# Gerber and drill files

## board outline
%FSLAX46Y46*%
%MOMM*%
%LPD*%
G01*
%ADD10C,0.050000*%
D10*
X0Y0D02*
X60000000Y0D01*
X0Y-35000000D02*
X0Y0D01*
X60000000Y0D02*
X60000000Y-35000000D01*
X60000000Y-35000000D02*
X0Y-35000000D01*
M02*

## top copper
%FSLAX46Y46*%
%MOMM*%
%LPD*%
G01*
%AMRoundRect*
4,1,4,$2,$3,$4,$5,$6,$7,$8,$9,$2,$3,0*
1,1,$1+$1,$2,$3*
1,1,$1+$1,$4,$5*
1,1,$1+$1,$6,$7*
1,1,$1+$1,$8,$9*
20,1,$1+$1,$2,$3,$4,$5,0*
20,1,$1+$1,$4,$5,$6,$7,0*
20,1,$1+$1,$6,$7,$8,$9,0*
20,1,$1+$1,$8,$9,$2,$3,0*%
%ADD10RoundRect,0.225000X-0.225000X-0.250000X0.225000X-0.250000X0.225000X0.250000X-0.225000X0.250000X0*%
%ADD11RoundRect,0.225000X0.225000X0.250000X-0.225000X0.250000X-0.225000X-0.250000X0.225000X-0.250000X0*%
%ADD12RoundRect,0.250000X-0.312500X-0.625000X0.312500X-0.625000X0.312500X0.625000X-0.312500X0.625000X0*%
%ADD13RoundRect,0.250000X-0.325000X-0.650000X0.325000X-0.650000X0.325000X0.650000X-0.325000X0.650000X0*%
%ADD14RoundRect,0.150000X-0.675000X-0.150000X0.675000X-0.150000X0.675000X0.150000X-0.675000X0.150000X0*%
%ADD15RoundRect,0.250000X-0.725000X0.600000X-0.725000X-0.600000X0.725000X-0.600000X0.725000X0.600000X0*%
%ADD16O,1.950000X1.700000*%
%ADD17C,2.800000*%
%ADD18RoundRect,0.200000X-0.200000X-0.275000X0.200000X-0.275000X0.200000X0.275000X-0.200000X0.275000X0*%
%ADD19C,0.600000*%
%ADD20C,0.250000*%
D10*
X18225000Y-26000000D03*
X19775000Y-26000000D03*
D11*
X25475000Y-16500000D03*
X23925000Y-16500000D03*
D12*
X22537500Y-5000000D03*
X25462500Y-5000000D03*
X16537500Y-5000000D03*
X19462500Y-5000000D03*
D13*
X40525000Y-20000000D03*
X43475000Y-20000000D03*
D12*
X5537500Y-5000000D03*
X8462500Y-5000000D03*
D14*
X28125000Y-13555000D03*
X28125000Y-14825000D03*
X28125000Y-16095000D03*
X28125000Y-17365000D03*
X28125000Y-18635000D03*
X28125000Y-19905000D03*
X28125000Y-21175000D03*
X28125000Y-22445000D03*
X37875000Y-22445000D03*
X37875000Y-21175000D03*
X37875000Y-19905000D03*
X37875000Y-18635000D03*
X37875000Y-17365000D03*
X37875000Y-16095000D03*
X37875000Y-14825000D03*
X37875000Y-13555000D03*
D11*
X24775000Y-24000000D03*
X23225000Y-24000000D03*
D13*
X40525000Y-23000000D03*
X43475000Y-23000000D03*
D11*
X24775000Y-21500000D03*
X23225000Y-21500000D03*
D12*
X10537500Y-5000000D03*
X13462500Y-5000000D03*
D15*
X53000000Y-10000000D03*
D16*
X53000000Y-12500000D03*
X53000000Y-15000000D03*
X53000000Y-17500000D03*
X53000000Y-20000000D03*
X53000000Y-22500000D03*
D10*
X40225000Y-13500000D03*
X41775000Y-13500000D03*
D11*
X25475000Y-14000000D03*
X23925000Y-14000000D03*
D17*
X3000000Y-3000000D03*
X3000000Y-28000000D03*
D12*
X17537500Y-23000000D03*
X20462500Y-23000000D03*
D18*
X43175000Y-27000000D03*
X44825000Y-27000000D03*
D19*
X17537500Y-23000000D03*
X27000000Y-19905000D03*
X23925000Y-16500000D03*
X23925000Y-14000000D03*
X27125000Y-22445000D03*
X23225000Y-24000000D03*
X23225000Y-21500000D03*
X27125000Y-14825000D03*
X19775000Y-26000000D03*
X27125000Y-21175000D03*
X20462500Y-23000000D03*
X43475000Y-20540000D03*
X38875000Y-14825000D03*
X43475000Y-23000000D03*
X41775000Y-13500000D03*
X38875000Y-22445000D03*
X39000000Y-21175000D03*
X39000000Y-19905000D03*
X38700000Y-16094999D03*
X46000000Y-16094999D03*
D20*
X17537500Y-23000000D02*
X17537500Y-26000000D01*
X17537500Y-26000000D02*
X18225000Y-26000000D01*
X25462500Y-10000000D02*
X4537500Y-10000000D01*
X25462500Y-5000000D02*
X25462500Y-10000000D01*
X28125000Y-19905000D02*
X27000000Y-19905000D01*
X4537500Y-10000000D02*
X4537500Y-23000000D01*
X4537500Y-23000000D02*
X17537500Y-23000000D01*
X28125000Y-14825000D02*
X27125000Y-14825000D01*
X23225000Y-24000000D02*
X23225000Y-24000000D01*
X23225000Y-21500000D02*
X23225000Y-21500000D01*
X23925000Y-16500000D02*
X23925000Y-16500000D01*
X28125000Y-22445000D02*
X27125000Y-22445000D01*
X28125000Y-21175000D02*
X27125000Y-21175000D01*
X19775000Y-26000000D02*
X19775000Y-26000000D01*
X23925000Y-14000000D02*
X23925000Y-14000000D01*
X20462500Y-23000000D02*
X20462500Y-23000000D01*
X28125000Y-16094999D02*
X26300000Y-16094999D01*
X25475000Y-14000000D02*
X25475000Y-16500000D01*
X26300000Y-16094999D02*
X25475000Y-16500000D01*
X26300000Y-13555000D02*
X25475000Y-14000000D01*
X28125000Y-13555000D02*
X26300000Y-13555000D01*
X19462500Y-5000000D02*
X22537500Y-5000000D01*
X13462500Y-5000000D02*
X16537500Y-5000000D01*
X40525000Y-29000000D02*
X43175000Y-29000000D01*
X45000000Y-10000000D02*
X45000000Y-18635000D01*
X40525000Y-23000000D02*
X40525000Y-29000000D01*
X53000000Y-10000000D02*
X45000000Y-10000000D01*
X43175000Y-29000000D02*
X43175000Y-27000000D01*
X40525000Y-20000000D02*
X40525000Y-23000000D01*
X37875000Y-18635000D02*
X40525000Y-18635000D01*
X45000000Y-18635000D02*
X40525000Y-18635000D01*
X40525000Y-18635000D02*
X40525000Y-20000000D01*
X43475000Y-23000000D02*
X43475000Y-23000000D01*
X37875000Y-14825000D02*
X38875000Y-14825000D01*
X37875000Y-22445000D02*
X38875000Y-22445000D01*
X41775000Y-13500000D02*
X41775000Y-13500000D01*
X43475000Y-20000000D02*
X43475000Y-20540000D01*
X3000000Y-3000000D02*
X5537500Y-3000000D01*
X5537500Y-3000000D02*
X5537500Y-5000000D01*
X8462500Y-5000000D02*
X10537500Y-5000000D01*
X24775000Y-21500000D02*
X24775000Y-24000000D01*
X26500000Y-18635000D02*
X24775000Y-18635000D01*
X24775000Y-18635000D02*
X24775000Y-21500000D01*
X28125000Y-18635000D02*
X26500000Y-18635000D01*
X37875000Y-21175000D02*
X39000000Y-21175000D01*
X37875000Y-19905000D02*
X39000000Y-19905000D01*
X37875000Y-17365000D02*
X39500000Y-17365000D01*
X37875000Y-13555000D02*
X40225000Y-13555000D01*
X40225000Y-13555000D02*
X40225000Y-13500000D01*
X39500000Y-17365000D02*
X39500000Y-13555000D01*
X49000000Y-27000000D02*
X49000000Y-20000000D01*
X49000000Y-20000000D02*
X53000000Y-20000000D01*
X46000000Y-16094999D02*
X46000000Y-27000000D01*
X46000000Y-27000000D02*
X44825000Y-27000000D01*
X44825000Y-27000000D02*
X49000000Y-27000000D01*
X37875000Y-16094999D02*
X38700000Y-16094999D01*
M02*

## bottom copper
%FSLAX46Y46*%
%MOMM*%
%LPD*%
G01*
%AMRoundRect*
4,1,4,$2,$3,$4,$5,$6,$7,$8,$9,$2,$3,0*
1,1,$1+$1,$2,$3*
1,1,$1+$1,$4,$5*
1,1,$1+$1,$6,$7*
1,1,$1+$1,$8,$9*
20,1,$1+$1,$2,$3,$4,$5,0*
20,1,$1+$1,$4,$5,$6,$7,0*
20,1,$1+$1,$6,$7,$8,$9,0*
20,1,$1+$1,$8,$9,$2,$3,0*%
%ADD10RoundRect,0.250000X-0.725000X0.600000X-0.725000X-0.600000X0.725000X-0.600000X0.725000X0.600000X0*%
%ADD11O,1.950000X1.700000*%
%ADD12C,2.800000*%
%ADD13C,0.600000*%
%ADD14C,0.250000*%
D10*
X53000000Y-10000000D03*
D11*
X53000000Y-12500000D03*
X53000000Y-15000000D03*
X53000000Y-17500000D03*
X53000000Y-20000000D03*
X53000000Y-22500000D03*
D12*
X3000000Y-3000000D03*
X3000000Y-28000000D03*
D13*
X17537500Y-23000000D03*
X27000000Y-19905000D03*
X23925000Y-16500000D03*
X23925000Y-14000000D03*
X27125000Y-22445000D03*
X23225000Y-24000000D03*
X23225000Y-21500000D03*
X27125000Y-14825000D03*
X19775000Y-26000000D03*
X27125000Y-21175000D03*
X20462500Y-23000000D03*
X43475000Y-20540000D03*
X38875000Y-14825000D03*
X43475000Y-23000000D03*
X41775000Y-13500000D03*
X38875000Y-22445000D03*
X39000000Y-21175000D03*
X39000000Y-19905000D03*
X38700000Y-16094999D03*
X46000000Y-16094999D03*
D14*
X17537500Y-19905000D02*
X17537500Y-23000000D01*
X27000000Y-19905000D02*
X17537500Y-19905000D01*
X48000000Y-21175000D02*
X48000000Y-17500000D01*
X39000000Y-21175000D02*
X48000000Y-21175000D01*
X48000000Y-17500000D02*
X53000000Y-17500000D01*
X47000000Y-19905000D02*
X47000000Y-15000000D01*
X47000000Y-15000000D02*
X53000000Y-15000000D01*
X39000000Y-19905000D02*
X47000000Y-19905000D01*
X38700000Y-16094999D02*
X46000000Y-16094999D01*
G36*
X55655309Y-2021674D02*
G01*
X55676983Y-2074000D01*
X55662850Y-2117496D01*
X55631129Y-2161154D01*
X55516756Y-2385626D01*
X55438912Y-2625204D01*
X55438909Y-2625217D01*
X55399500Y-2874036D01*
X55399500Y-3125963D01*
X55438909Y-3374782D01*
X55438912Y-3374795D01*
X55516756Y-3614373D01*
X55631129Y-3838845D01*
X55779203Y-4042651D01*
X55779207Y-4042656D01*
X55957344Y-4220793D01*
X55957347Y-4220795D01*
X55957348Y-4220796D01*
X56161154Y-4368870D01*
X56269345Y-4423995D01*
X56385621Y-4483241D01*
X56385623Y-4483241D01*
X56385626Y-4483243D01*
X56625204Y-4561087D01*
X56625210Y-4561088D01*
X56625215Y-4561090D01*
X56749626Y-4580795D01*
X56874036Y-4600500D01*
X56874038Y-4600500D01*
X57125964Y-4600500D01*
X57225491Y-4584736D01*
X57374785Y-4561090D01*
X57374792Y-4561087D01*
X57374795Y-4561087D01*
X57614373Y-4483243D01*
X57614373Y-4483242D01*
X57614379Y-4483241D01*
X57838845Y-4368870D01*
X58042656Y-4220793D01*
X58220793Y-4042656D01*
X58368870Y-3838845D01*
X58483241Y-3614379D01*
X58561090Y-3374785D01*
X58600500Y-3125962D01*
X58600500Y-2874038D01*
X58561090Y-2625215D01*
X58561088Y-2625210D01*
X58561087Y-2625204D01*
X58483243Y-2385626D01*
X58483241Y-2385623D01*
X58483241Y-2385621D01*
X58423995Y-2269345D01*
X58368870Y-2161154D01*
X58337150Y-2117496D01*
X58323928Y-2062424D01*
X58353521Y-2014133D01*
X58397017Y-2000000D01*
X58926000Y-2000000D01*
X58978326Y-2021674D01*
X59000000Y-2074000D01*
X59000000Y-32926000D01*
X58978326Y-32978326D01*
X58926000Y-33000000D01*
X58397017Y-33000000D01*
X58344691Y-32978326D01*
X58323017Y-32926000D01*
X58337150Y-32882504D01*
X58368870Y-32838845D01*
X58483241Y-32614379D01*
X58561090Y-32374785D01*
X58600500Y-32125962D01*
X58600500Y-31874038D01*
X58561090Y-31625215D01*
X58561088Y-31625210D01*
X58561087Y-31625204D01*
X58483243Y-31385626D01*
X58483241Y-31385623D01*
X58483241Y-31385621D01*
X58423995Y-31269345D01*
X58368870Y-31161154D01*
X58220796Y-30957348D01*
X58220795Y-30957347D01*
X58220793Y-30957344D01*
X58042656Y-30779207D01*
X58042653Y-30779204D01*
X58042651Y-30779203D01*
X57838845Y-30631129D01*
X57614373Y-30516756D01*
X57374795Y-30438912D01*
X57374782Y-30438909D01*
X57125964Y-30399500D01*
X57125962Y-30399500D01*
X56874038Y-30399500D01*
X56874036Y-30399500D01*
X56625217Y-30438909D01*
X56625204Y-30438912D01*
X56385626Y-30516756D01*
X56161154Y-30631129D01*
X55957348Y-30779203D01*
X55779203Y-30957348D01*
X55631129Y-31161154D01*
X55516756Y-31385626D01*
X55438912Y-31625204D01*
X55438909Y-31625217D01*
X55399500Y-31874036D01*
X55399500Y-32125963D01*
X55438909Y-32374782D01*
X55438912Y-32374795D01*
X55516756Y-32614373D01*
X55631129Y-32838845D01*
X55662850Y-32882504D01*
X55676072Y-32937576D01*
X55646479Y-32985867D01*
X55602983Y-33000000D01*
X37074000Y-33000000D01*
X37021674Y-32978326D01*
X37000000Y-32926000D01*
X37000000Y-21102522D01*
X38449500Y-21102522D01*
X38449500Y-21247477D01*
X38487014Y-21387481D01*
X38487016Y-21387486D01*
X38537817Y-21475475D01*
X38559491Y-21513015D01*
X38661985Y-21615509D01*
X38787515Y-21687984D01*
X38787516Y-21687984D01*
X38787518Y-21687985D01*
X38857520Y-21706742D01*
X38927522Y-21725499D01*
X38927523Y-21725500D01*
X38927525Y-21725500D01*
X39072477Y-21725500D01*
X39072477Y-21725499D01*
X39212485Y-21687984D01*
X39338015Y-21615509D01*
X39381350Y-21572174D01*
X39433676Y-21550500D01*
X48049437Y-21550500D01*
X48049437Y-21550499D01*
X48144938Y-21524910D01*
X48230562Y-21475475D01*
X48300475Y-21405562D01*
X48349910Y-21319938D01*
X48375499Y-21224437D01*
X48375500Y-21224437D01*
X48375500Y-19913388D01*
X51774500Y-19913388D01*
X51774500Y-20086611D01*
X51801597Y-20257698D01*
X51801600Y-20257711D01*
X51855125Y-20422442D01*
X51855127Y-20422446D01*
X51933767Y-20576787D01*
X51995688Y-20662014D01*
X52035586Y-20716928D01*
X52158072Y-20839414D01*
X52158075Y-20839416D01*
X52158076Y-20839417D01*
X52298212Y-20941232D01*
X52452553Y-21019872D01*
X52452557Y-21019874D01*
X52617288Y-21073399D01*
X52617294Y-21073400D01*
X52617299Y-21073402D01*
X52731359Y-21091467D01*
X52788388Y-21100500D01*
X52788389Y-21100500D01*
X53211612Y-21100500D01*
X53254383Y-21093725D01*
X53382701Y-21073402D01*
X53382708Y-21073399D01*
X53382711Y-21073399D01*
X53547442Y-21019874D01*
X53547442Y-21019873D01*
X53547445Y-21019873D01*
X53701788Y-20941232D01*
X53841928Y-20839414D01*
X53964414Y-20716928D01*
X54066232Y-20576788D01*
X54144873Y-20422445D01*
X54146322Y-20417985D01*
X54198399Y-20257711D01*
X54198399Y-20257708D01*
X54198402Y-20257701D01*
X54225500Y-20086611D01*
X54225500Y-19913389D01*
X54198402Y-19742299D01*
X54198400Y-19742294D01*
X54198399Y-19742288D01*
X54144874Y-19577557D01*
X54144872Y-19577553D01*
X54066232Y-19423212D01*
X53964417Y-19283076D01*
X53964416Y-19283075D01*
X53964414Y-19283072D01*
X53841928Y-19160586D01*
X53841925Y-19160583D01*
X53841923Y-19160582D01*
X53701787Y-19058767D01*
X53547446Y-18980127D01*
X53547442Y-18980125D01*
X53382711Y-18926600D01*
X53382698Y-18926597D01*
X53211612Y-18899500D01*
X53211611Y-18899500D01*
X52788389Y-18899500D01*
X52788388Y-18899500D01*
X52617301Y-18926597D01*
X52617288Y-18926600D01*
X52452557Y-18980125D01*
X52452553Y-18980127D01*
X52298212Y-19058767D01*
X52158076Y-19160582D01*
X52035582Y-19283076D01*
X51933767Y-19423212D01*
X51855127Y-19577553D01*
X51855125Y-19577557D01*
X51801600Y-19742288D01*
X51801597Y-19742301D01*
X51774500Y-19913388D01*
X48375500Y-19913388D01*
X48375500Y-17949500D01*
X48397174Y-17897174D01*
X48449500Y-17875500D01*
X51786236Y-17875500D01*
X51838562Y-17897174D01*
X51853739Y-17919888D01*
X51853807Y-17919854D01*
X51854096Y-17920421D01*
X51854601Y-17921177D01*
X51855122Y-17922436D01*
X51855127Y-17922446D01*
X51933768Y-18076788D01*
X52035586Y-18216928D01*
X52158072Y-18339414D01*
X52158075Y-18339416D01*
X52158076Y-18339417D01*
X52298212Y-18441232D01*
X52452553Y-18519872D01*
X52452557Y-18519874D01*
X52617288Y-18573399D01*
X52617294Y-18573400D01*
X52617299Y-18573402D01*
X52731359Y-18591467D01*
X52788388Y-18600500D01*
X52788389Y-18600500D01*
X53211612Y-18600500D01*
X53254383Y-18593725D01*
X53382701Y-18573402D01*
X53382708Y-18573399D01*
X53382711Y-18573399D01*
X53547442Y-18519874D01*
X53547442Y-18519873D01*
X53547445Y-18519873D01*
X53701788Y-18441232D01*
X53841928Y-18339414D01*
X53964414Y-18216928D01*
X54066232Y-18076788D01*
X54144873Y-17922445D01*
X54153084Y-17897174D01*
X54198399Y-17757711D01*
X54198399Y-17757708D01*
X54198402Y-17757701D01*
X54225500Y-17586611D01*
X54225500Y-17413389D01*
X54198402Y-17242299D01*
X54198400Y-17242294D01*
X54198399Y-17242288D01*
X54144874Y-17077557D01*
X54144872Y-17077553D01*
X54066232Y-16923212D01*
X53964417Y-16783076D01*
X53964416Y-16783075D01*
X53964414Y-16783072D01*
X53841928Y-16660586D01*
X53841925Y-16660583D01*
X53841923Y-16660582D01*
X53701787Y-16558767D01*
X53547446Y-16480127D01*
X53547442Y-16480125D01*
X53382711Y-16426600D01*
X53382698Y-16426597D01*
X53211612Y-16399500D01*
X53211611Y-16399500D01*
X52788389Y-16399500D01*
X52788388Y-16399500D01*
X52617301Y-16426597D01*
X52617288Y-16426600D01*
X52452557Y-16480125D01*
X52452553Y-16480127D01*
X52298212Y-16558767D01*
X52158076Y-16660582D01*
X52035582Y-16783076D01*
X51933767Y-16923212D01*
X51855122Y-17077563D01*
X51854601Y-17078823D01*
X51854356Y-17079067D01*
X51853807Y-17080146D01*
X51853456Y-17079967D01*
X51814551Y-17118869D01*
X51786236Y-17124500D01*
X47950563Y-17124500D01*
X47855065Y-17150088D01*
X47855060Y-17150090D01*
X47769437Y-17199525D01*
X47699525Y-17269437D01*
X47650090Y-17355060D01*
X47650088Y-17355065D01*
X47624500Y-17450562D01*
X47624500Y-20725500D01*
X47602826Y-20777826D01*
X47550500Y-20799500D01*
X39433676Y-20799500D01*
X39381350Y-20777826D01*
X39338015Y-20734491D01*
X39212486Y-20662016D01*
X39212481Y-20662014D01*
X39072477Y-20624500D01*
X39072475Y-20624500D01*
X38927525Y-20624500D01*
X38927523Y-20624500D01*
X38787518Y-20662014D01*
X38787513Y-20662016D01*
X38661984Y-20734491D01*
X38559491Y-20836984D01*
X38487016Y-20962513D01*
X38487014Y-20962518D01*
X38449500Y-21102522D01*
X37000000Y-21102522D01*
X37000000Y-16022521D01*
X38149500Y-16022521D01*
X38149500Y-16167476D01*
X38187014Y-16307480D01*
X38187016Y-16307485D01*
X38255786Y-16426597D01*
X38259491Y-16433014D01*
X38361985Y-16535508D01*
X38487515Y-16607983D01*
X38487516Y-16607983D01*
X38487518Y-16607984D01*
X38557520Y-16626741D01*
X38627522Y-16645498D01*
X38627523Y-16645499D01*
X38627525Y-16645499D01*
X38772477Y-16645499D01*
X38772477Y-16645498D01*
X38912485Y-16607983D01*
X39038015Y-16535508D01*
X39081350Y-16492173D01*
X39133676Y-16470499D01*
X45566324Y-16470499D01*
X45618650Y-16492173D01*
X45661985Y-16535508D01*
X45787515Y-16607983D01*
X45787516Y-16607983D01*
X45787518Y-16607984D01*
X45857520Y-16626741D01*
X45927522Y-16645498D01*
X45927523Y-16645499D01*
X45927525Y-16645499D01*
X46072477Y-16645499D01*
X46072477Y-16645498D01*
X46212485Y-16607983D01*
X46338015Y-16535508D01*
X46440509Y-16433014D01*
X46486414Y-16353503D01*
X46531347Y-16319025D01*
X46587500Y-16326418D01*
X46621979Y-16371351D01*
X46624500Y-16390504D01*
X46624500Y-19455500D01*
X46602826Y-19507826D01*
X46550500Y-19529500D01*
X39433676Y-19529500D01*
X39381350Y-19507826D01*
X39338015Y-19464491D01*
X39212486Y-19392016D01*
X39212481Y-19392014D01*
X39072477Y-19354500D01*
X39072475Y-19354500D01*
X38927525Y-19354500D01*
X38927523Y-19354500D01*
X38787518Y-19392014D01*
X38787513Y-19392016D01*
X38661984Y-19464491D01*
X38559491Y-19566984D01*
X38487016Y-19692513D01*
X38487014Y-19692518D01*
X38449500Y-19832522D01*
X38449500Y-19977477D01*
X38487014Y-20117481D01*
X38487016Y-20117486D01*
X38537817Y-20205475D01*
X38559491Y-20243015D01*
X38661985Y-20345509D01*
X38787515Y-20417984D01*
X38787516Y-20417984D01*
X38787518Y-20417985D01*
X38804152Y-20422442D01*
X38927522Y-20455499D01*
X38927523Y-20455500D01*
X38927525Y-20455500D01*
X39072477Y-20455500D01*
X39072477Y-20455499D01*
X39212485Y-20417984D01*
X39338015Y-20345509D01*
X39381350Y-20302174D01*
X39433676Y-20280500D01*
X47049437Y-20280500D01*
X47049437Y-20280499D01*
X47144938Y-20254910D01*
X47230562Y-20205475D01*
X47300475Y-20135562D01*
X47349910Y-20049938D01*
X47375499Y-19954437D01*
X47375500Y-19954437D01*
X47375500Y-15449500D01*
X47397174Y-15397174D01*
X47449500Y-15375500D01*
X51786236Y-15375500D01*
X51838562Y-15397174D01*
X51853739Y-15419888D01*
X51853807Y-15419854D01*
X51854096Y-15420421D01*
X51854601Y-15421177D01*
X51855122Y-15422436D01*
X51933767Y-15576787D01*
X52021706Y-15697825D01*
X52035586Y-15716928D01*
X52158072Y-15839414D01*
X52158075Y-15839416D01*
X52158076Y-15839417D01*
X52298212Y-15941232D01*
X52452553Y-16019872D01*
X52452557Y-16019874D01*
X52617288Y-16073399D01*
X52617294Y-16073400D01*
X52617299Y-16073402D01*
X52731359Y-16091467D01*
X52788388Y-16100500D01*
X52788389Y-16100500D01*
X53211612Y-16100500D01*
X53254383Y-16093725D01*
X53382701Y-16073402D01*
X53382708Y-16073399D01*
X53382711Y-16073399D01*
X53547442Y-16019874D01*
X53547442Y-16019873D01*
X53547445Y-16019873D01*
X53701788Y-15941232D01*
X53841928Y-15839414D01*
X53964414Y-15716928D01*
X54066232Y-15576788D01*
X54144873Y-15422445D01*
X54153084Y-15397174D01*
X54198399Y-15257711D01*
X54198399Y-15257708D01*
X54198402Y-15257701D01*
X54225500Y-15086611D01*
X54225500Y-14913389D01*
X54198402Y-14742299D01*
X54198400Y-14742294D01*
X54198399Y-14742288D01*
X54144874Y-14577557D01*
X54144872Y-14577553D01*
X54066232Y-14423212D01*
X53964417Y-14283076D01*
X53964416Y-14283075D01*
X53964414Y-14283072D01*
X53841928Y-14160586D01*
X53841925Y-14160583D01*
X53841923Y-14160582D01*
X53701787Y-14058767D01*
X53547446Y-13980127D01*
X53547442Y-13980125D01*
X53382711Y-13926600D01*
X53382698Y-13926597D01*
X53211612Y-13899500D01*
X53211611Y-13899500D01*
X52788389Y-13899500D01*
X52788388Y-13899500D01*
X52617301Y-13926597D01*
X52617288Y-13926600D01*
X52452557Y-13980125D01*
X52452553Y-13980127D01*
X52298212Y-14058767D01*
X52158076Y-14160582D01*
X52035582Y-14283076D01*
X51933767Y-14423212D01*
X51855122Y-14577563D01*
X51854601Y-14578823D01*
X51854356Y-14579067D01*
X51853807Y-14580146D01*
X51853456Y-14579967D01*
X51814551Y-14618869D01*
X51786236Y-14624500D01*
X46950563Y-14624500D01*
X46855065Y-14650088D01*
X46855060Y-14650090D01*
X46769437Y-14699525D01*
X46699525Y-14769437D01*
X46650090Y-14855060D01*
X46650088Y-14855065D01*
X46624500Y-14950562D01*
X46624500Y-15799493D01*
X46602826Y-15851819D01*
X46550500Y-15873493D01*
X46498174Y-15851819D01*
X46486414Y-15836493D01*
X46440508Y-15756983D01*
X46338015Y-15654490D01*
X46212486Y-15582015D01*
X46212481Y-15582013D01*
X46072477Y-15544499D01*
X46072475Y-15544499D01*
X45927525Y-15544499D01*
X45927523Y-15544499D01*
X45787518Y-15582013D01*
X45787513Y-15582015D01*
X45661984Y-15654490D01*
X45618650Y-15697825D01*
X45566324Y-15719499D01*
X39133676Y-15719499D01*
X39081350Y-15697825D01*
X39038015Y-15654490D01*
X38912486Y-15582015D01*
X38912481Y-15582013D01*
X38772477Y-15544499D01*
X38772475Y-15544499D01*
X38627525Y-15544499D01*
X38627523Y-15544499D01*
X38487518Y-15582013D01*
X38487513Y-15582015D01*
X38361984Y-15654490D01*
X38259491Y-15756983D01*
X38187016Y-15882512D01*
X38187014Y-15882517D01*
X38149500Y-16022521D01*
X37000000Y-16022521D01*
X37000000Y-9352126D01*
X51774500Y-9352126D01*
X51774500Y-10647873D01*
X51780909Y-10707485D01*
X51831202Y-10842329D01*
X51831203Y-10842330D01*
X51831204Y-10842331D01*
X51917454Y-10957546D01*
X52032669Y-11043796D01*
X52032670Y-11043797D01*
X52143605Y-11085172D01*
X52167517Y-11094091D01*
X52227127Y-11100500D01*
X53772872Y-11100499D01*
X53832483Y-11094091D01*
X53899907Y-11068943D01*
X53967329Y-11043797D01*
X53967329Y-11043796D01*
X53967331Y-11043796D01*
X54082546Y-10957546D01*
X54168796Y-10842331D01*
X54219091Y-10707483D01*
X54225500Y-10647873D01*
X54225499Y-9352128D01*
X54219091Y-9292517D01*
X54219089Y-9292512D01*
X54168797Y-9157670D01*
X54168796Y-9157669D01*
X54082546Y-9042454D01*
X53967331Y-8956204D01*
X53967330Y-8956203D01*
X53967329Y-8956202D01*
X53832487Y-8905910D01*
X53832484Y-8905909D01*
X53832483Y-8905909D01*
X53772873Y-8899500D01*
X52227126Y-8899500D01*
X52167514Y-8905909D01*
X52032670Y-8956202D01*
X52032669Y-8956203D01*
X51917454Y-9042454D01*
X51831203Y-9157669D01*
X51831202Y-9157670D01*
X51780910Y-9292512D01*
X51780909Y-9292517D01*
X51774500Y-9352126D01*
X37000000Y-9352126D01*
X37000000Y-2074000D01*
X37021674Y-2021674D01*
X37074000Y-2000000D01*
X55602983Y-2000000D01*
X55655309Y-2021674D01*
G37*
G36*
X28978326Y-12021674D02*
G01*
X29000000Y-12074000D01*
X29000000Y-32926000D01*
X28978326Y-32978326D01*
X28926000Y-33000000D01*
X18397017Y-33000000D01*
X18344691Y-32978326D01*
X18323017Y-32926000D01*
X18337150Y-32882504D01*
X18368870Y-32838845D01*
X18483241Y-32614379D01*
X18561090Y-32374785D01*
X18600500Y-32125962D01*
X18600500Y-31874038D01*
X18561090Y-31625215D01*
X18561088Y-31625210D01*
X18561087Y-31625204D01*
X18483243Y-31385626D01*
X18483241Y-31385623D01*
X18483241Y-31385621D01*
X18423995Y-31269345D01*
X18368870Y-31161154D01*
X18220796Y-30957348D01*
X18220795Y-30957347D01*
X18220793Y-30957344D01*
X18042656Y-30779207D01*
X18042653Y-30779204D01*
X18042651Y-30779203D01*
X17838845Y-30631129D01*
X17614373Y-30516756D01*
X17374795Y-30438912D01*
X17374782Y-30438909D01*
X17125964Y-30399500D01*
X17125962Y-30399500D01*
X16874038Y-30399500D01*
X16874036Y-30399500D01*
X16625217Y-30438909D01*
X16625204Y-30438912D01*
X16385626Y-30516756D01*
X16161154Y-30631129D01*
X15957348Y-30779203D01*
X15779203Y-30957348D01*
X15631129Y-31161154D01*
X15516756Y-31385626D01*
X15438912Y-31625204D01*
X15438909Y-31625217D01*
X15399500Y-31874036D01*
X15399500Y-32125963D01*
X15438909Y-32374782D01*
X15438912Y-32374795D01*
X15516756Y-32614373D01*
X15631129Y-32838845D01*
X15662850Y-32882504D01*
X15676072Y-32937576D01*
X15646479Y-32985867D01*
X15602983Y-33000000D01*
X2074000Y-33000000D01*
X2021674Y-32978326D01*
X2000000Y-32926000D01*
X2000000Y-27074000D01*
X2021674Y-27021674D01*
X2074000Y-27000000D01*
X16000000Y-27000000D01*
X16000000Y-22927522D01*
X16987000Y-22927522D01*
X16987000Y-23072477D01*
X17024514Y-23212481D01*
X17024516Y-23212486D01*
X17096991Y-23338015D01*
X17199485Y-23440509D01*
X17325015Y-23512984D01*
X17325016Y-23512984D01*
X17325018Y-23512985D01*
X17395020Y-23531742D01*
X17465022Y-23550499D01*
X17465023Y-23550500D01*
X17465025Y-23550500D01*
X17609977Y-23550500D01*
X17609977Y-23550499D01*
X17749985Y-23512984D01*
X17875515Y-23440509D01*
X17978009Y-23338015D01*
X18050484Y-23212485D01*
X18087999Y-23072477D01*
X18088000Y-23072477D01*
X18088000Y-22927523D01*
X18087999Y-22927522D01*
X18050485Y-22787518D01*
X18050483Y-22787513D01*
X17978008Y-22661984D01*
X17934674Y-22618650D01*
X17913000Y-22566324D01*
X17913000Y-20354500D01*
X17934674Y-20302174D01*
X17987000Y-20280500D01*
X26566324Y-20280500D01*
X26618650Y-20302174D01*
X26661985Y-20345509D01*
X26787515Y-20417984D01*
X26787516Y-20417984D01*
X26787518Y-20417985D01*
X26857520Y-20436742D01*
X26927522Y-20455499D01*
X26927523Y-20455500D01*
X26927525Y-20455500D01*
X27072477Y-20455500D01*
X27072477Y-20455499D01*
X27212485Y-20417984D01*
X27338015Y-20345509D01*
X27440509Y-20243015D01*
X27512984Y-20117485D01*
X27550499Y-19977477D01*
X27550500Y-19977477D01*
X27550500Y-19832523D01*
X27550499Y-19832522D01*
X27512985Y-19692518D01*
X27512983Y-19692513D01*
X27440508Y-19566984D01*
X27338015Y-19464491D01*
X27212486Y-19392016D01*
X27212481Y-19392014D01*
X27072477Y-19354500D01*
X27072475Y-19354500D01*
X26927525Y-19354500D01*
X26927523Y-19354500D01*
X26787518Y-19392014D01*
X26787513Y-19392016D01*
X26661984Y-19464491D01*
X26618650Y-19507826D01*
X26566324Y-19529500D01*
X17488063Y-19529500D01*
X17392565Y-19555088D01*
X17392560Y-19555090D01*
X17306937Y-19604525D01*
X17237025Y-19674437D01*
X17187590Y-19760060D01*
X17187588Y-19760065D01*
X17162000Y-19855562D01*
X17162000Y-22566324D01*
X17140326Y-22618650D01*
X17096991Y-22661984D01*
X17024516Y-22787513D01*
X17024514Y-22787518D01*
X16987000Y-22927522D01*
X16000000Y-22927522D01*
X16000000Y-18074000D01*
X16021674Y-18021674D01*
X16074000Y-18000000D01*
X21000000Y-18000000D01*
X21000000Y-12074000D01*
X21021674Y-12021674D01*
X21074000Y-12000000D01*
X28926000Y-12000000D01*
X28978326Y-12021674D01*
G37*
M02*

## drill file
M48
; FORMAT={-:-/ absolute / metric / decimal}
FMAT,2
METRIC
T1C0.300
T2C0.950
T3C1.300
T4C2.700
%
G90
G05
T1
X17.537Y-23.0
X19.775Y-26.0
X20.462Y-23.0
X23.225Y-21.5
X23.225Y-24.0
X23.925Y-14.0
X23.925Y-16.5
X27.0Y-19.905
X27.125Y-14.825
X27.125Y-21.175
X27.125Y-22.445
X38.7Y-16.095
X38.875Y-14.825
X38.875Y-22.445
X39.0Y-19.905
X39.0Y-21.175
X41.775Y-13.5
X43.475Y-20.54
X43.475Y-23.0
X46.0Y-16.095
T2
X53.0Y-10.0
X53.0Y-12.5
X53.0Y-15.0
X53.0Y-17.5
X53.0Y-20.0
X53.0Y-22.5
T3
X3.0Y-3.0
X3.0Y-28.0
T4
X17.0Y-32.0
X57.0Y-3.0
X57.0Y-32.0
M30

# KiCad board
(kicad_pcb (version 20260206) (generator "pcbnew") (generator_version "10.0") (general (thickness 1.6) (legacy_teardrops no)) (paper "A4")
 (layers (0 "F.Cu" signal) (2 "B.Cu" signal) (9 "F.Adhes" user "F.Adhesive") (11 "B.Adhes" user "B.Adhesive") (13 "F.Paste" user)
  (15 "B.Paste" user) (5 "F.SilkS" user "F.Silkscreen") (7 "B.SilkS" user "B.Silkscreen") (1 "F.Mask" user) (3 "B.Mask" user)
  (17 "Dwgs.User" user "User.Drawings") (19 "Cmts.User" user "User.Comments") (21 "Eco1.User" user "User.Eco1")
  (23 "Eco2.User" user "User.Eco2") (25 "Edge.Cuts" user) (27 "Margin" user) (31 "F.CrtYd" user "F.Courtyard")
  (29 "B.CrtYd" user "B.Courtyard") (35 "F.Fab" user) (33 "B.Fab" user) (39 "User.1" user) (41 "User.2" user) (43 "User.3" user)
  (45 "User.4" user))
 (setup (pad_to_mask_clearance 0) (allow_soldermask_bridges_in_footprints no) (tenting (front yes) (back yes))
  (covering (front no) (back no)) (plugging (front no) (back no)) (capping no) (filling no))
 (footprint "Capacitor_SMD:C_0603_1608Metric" (layer "F.Cu") (at 19 26)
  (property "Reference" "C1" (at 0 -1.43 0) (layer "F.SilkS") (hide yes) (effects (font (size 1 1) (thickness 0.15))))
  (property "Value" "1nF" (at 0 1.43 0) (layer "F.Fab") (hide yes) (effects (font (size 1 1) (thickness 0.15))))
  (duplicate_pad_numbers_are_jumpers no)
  (pad "1" smd roundrect (at -0.775 0) (size 0.9 0.95) (layers "F.Cu" "F.Mask" "F.Paste") (roundrect_rratio 0.25) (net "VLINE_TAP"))
  (pad "2" smd roundrect (at 0.775 0) (size 0.9 0.95) (layers "F.Cu" "F.Mask" "F.Paste") (roundrect_rratio 0.25) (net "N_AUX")))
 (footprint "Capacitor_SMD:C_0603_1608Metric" (layer "F.Cu") (at 24.7 16.5 180)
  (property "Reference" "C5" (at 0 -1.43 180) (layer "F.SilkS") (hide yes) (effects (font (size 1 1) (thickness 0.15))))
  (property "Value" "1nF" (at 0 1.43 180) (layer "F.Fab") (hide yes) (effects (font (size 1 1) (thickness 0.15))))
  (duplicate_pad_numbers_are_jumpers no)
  (pad "1" smd roundrect (at -0.775 0 180) (size 0.9 0.95) (layers "F.Cu" "F.Mask" "F.Paste") (roundrect_rratio 0.25) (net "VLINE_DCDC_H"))
  (pad "2" smd roundrect (at 0.775 0 180) (size 0.9 0.95) (layers "F.Cu" "F.Mask" "F.Paste") (roundrect_rratio 0.25) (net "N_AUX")))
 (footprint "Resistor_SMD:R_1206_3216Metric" (layer "F.Cu") (at 24 5)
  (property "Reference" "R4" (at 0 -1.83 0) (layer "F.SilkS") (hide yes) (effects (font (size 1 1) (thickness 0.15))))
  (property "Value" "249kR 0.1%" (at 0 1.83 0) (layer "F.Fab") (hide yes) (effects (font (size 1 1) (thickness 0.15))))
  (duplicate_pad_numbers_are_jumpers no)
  (pad "1" smd roundrect (at -1.4625 0) (size 1.125 1.75) (layers "F.Cu" "F.Mask" "F.Paste") (roundrect_rratio 0.222222) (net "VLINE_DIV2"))
  (pad "2" smd roundrect (at 1.4625 0) (size 1.125 1.75) (layers "F.Cu" "F.Mask" "F.Paste") (roundrect_rratio 0.222222) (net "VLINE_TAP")))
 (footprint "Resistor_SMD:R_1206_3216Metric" (layer "F.Cu") (at 18 5)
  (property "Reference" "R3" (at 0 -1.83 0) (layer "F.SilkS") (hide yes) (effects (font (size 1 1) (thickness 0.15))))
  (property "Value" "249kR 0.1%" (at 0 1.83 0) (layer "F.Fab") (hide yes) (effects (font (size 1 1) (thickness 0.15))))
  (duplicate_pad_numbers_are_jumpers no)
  (pad "1" smd roundrect (at -1.4625 0) (size 1.125 1.75) (layers "F.Cu" "F.Mask" "F.Paste") (roundrect_rratio 0.222222) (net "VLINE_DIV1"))
  (pad "2" smd roundrect (at 1.4625 0) (size 1.125 1.75) (layers "F.Cu" "F.Mask" "F.Paste") (roundrect_rratio 0.222222) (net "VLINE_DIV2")))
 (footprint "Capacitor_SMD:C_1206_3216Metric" (layer "F.Cu") (at 42 20)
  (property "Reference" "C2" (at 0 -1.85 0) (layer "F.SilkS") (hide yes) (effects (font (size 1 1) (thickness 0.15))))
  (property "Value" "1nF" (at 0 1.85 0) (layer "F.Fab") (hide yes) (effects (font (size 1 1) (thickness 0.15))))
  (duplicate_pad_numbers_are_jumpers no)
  (pad "1" smd roundrect (at -1.475 0) (size 1.15 1.8) (layers "F.Cu" "F.Mask" "F.Paste") (roundrect_rratio 0.217391) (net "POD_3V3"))
  (pad "2" smd roundrect (at 1.475 0) (size 1.15 1.8) (layers "F.Cu" "F.Mask" "F.Paste") (roundrect_rratio 0.217391) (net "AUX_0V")))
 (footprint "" (layer "F.Cu") (at 57 32)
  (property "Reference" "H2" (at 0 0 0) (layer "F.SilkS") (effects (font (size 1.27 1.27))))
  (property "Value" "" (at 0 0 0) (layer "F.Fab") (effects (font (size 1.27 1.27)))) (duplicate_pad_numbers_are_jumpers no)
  (pad "" np_thru_hole circle (at 0 0) (size 2.7 2.7) (drill 2.7) (layers "*.Cu")))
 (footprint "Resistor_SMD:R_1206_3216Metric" (layer "F.Cu") (at 7 5)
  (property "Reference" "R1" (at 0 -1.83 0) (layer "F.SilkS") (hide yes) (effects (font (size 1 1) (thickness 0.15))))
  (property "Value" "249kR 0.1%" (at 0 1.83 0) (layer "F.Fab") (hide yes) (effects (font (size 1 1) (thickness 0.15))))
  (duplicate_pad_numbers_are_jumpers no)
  (pad "1" smd roundrect (at -1.4625 0) (size 1.125 1.75) (layers "F.Cu" "F.Mask" "F.Paste") (roundrect_rratio 0.222222) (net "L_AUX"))
  (pad "2" smd roundrect (at 1.4625 0) (size 1.125 1.75) (layers "F.Cu" "F.Mask" "F.Paste") (roundrect_rratio 0.222222) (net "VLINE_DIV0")))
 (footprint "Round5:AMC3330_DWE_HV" (layer "F.Cu") (at 33 18)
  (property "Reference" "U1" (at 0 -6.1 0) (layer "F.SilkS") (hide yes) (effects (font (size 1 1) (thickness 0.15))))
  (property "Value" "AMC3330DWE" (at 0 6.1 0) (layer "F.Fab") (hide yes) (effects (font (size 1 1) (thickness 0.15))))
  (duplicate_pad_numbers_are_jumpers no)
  (pad "1" smd roundrect (at -4.875 -4.445) (size 1.65 0.6) (layers "F.Cu" "F.Mask" "F.Paste") (roundrect_rratio 0.25) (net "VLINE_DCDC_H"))
  (pad "2" smd roundrect (at -4.875 -3.175) (size 1.65 0.6) (layers "F.Cu" "F.Mask" "F.Paste") (roundrect_rratio 0.25) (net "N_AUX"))
  (pad "3" smd roundrect (at -4.875 -1.905) (size 1.65 0.6) (layers "F.Cu" "F.Mask" "F.Paste") (roundrect_rratio 0.25) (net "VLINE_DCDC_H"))
  (pad "4" smd roundrect (at -4.875 -0.635) (size 1.65 0.6) (layers "F.Cu" "F.Mask" "F.Paste") (roundrect_rratio 0.25)
   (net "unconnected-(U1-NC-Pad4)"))
  (pad "5" smd roundrect (at -4.875 0.635) (size 1.65 0.6) (layers "F.Cu" "F.Mask" "F.Paste") (roundrect_rratio 0.25) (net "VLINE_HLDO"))
  (pad "6" smd roundrect (at -4.875 1.905) (size 1.65 0.6) (layers "F.Cu" "F.Mask" "F.Paste") (roundrect_rratio 0.25) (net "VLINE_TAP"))
  (pad "7" smd roundrect (at -4.875 3.175) (size 1.65 0.6) (layers "F.Cu" "F.Mask" "F.Paste") (roundrect_rratio 0.25) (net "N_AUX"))
  (pad "8" smd roundrect (at -4.875 4.445) (size 1.65 0.6) (layers "F.Cu" "F.Mask" "F.Paste") (roundrect_rratio 0.25) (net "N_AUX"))
  (pad "9" smd roundrect (at 4.875 4.445) (size 1.65 0.6) (layers "F.Cu" "F.Mask" "F.Paste") (roundrect_rratio 0.25) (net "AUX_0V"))
  (pad "10" smd roundrect (at 4.875 3.175) (size 1.65 0.6) (layers "F.Cu" "F.Mask" "F.Paste") (roundrect_rratio 0.25) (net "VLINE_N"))
  (pad "11" smd roundrect (at 4.875 1.905) (size 1.65 0.6) (layers "F.Cu" "F.Mask" "F.Paste") (roundrect_rratio 0.25) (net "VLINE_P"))
  (pad "12" smd roundrect (at 4.875 0.635) (size 1.65 0.6) (layers "F.Cu" "F.Mask" "F.Paste") (roundrect_rratio 0.25) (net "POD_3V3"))
  (pad "13" smd roundrect (at 4.875 -0.635) (size 1.65 0.6) (layers "F.Cu" "F.Mask" "F.Paste") (roundrect_rratio 0.25) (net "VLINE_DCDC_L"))
  (pad "14" smd roundrect (at 4.875 -1.905) (size 1.65 0.6) (layers "F.Cu" "F.Mask" "F.Paste") (roundrect_rratio 0.25) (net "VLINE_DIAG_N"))
  (pad "15" smd roundrect (at 4.875 -3.175) (size 1.65 0.6) (layers "F.Cu" "F.Mask" "F.Paste") (roundrect_rratio 0.25) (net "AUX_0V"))
  (pad "16" smd roundrect (at 4.875 -4.445) (size 1.65 0.6) (layers "F.Cu" "F.Mask" "F.Paste") (roundrect_rratio 0.25) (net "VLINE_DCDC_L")))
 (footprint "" (layer "F.Cu") (at 17 32)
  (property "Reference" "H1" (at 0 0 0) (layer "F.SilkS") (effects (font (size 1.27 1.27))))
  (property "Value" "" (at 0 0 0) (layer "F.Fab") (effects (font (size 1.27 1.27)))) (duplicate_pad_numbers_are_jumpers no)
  (pad "" np_thru_hole circle (at 0 0) (size 2.7 2.7) (drill 2.7) (layers "*.Cu")))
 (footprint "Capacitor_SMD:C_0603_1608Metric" (layer "F.Cu") (at 24 24 180)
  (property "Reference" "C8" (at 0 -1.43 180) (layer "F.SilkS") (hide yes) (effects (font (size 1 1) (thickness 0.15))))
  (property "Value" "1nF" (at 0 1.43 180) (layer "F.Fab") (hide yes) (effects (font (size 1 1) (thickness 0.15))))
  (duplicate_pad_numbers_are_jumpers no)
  (pad "1" smd roundrect (at -0.775 0 180) (size 0.9 0.95) (layers "F.Cu" "F.Mask" "F.Paste") (roundrect_rratio 0.25) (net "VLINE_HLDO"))
  (pad "2" smd roundrect (at 0.775 0 180) (size 0.9 0.95) (layers "F.Cu" "F.Mask" "F.Paste") (roundrect_rratio 0.25) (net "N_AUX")))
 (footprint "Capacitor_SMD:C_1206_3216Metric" (layer "F.Cu") (at 42 23)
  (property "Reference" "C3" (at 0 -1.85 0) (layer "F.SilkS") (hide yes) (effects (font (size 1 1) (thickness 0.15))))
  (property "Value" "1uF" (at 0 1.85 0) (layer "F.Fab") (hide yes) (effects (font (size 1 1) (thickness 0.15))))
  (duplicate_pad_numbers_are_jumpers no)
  (pad "1" smd roundrect (at -1.475 0) (size 1.15 1.8) (layers "F.Cu" "F.Mask" "F.Paste") (roundrect_rratio 0.217391) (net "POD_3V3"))
  (pad "2" smd roundrect (at 1.475 0) (size 1.15 1.8) (layers "F.Cu" "F.Mask" "F.Paste") (roundrect_rratio 0.217391) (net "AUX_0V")))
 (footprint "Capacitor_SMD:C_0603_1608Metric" (layer "F.Cu") (at 24 21.5 180)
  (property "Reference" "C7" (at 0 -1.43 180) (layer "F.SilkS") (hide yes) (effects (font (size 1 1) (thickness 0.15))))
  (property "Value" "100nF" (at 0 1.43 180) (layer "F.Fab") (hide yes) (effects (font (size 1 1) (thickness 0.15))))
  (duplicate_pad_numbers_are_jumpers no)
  (pad "1" smd roundrect (at -0.775 0 180) (size 0.9 0.95) (layers "F.Cu" "F.Mask" "F.Paste") (roundrect_rratio 0.25) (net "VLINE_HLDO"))
  (pad "2" smd roundrect (at 0.775 0 180) (size 0.9 0.95) (layers "F.Cu" "F.Mask" "F.Paste") (roundrect_rratio 0.25) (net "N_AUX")))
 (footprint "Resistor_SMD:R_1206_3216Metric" (layer "F.Cu") (at 12 5)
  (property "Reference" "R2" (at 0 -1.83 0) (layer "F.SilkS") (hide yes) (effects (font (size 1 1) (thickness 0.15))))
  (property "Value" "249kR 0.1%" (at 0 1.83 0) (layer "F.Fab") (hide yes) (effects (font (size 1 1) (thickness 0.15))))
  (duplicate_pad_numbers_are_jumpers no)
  (pad "1" smd roundrect (at -1.4625 0) (size 1.125 1.75) (layers "F.Cu" "F.Mask" "F.Paste") (roundrect_rratio 0.222222) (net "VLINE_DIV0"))
  (pad "2" smd roundrect (at 1.4625 0) (size 1.125 1.75) (layers "F.Cu" "F.Mask" "F.Paste") (roundrect_rratio 0.222222) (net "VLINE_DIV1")))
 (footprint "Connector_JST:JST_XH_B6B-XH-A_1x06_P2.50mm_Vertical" (layer "F.Cu") (at 53 10 -90)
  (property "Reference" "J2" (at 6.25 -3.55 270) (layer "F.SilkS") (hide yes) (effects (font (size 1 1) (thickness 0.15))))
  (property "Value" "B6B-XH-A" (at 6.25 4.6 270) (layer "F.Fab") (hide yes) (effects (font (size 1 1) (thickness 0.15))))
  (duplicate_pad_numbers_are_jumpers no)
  (pad "1" thru_hole roundrect (at 0 0 270) (size 1.7 1.95) (drill 0.95) (layers "*.Cu" "*.Mask") (remove_unused_layers no)
   (roundrect_rratio 0.147059) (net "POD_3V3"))
  (pad "2" thru_hole oval (at 2.5 0 270) (size 1.7 1.95) (drill 0.95) (layers "*.Cu" "*.Mask") (remove_unused_layers no) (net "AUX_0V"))
  (pad "3" thru_hole oval (at 5 0 270) (size 1.7 1.95) (drill 0.95) (layers "*.Cu" "*.Mask") (remove_unused_layers no) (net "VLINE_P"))
  (pad "4" thru_hole oval (at 7.5 0 270) (size 1.7 1.95) (drill 0.95) (layers "*.Cu" "*.Mask") (remove_unused_layers no) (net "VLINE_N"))
  (pad "5" thru_hole oval (at 10 0 270) (size 1.7 1.95) (drill 0.95) (layers "*.Cu" "*.Mask") (remove_unused_layers no) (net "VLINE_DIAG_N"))
  (pad "6" thru_hole oval (at 12.5 0 270) (size 1.7 1.95) (drill 0.95) (layers "*.Cu" "*.Mask") (remove_unused_layers no) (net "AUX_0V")))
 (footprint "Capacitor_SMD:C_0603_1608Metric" (layer "F.Cu") (at 41 13.5)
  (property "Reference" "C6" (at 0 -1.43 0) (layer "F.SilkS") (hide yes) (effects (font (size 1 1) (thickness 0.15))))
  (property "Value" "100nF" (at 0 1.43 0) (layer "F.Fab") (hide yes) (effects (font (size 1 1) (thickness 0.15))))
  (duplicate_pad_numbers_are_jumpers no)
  (pad "1" smd roundrect (at -0.775 0) (size 0.9 0.95) (layers "F.Cu" "F.Mask" "F.Paste") (roundrect_rratio 0.25) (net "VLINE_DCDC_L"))
  (pad "2" smd roundrect (at 0.775 0) (size 0.9 0.95) (layers "F.Cu" "F.Mask" "F.Paste") (roundrect_rratio 0.25) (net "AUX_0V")))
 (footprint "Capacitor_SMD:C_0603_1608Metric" (layer "F.Cu") (at 24.7 14 180)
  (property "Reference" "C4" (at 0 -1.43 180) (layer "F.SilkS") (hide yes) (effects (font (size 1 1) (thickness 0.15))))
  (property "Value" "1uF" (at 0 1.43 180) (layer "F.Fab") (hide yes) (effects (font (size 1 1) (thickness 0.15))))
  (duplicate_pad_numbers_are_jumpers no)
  (pad "1" smd roundrect (at -0.775 0 180) (size 0.9 0.95) (layers "F.Cu" "F.Mask" "F.Paste") (roundrect_rratio 0.25) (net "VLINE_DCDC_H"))
  (pad "2" smd roundrect (at 0.775 0 180) (size 0.9 0.95) (layers "F.Cu" "F.Mask" "F.Paste") (roundrect_rratio 0.25) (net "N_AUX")))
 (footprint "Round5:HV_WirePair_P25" (layer "F.Cu") (at 3 3)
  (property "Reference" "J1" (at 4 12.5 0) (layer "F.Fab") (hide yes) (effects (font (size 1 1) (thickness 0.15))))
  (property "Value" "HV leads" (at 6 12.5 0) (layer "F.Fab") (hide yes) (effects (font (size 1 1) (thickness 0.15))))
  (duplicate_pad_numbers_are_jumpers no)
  (pad "1" thru_hole circle (at 0 0) (size 2.8 2.8) (drill 1.3) (layers "*.Cu" "*.Mask") (remove_unused_layers no) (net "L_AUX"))
  (pad "2" thru_hole circle (at 0 25) (size 2.8 2.8) (drill 1.3) (layers "*.Cu" "*.Mask") (remove_unused_layers no) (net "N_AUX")))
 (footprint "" (layer "F.Cu") (at 57 3)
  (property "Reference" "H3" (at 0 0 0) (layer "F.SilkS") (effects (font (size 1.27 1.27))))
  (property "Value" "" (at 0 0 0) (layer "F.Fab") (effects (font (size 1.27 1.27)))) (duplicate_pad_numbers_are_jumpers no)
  (pad "" np_thru_hole circle (at 0 0) (size 2.7 2.7) (drill 2.7) (layers "*.Cu")))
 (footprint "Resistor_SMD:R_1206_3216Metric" (layer "F.Cu") (at 19 23)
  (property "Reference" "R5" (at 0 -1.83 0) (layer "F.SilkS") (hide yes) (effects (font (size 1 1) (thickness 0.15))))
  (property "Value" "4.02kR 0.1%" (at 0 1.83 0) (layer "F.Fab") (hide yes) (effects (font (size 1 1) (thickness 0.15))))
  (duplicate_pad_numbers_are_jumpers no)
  (pad "1" smd roundrect (at -1.4625 0) (size 1.125 1.75) (layers "F.Cu" "F.Mask" "F.Paste") (roundrect_rratio 0.222222) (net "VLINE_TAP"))
  (pad "2" smd roundrect (at 1.4625 0) (size 1.125 1.75) (layers "F.Cu" "F.Mask" "F.Paste") (roundrect_rratio 0.222222) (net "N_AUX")))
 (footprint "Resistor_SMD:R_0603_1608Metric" (layer "F.Cu") (at 44 27)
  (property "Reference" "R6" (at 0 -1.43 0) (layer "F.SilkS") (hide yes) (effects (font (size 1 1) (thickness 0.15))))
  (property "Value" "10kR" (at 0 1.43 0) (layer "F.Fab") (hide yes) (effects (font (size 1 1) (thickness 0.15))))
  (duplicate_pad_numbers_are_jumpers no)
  (pad "1" smd roundrect (at -0.825 0) (size 0.8 0.95) (layers "F.Cu" "F.Mask" "F.Paste") (roundrect_rratio 0.25) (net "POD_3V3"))
  (pad "2" smd roundrect (at 0.825 0) (size 0.8 0.95) (layers "F.Cu" "F.Mask" "F.Paste") (roundrect_rratio 0.25) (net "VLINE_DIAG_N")))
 (gr_line (start 0 0) (end 60 0) (stroke (width 0.05) (type default)) (layer "Edge.Cuts"))
 (gr_line (start 0 35) (end 0 0) (stroke (width 0.05) (type default)) (layer "Edge.Cuts"))
 (gr_line (start 60 0) (end 60 35) (stroke (width 0.05) (type default)) (layer "Edge.Cuts"))
 (gr_line (start 60 35) (end 0 35) (stroke (width 0.05) (type default)) (layer "Edge.Cuts"))
 (segment (start 17.5375 23) (end 17.5375 26) (width 0.25) (layer "F.Cu") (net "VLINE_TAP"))
 (segment (start 17.5375 26) (end 18.225 26) (width 0.25) (layer "F.Cu") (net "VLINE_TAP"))
 (segment (start 25.4625 10) (end 4.5375 10) (width 0.25) (layer "F.Cu") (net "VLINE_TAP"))
 (segment (start 25.4625 5) (end 25.4625 10) (width 0.25) (layer "F.Cu") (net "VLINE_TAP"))
 (segment (start 28.125 19.905) (end 27 19.905) (width 0.25) (layer "F.Cu") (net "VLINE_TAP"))
 (segment (start 4.5375 10) (end 4.5375 23) (width 0.25) (layer "F.Cu") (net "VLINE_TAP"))
 (segment (start 4.5375 23) (end 17.5375 23) (width 0.25) (layer "F.Cu") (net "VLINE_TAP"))
 (via (at 17.5375 23) (size 0.6) (drill 0.3) (layers "F.Cu" "B.Cu") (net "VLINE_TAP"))
 (via (at 27 19.905) (size 0.6) (drill 0.3) (layers "F.Cu" "B.Cu") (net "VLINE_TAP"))
 (segment (start 17.5375 19.905) (end 17.5375 23) (width 0.25) (layer "B.Cu") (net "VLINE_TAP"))
 (segment (start 27 19.905) (end 17.5375 19.905) (width 0.25) (layer "B.Cu") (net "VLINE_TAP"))
 (segment (start 28.125 14.825) (end 27.125 14.825) (width 0.25) (layer "F.Cu") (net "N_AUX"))
 (segment (start 23.225 24) (end 23.225 24) (width 0.25) (layer "F.Cu") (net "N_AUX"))
 (segment (start 23.225 21.5) (end 23.225 21.5) (width 0.25) (layer "F.Cu") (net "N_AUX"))
 (segment (start 23.925 16.5) (end 23.925 16.5) (width 0.25) (layer "F.Cu") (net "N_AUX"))
 (segment (start 28.125 22.445) (end 27.125 22.445) (width 0.25) (layer "F.Cu") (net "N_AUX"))
 (segment (start 28.125 21.175) (end 27.125 21.175) (width 0.25) (layer "F.Cu") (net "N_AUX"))
 (segment (start 19.775 26) (end 19.775 26) (width 0.25) (layer "F.Cu") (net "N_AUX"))
 (segment (start 23.925 14) (end 23.925 14) (width 0.25) (layer "F.Cu") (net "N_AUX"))
 (segment (start 20.4625 23) (end 20.4625 23) (width 0.25) (layer "F.Cu") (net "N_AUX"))
 (via (at 23.925 16.5) (size 0.6) (drill 0.3) (layers "F.Cu" "B.Cu") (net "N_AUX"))
 (via (at 23.925 14) (size 0.6) (drill 0.3) (layers "F.Cu" "B.Cu") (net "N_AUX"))
 (via (at 27.125 22.445) (size 0.6) (drill 0.3) (layers "F.Cu" "B.Cu") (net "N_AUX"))
 (via (at 23.225 24) (size 0.6) (drill 0.3) (layers "F.Cu" "B.Cu") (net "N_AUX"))
 (via (at 23.225 21.5) (size 0.6) (drill 0.3) (layers "F.Cu" "B.Cu") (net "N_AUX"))
 (via (at 27.125 14.825) (size 0.6) (drill 0.3) (layers "F.Cu" "B.Cu") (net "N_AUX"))
 (via (at 19.775 26) (size 0.6) (drill 0.3) (layers "F.Cu" "B.Cu") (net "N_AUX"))
 (via (at 27.125 21.175) (size 0.6) (drill 0.3) (layers "F.Cu" "B.Cu") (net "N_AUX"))
 (via (at 20.4625 23) (size 0.6) (drill 0.3) (layers "F.Cu" "B.Cu") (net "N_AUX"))
 (segment (start 28.125 16.094999) (end 26.3 16.094999) (width 0.25) (layer "F.Cu") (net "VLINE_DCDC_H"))
 (segment (start 25.475 14) (end 25.475 16.5) (width 0.25) (layer "F.Cu") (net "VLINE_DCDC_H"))
 (segment (start 26.3 16.094999) (end 25.475 16.5) (width 0.25) (layer "F.Cu") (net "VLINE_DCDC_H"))
 (segment (start 26.3 13.555) (end 25.475 14) (width 0.25) (layer "F.Cu") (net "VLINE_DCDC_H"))
 (segment (start 28.125 13.555) (end 26.3 13.555) (width 0.25) (layer "F.Cu") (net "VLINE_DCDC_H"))
 (segment (start 19.4625 5) (end 22.5375 5) (width 0.25) (layer "F.Cu") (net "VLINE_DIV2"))
 (segment (start 13.4625 5) (end 16.5375 5) (width 0.25) (layer "F.Cu") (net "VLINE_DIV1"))
 (segment (start 40.525 29) (end 43.175 29) (width 0.25) (layer "F.Cu") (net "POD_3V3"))
 (segment (start 45 10) (end 45 18.635) (width 0.25) (layer "F.Cu") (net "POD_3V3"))
 (segment (start 40.525 23) (end 40.525 29) (width 0.25) (layer "F.Cu") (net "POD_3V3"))
 (segment (start 53 10) (end 45 10) (width 0.25) (layer "F.Cu") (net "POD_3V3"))
 (segment (start 43.175 29) (end 43.175 27) (width 0.25) (layer "F.Cu") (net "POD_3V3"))
 (segment (start 40.525 20) (end 40.525 23) (width 0.25) (layer "F.Cu") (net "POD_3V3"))
 (segment (start 37.875 18.635) (end 40.525 18.635) (width 0.25) (layer "F.Cu") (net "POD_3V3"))
 (segment (start 45 18.635) (end 40.525 18.635) (width 0.25) (layer "F.Cu") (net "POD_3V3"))
 (segment (start 40.525 18.635) (end 40.525 20) (width 0.25) (layer "F.Cu") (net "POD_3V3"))
 (segment (start 43.475 23) (end 43.475 23) (width 0.25) (layer "F.Cu") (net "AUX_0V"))
 (segment (start 37.875 14.825) (end 38.875 14.825) (width 0.25) (layer "F.Cu") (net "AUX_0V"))
 (segment (start 37.875 22.445) (end 38.875 22.445) (width 0.25) (layer "F.Cu") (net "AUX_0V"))
 (segment (start 41.775 13.5) (end 41.775 13.5) (width 0.25) (layer "F.Cu") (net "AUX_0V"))
 (segment (start 43.475 20) (end 43.475 20.54) (width 0.25) (layer "F.Cu") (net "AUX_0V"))
 (via (at 43.475 20.54) (size 0.6) (drill 0.3) (layers "F.Cu" "B.Cu") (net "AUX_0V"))
 (via (at 38.875 14.825) (size 0.6) (drill 0.3) (layers "F.Cu" "B.Cu") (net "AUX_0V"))
 (via (at 43.475 23) (size 0.6) (drill 0.3) (layers "F.Cu" "B.Cu") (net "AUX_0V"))
 (via (at 41.775 13.5) (size 0.6) (drill 0.3) (layers "F.Cu" "B.Cu") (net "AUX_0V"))
 (via (at 38.875 22.445) (size 0.6) (drill 0.3) (layers "F.Cu" "B.Cu") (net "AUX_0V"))
 (segment (start 3 3) (end 5.5375 3) (width 0.25) (layer "F.Cu") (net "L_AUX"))
 (segment (start 5.5375 3) (end 5.5375 5) (width 0.25) (layer "F.Cu") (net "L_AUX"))
 (segment (start 8.4625 5) (end 10.5375 5) (width 0.25) (layer "F.Cu") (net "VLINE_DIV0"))
 (segment (start 24.775 21.5) (end 24.775 24) (width 0.25) (layer "F.Cu") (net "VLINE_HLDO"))
 (segment (start 26.5 18.635) (end 24.775 18.635) (width 0.25) (layer "F.Cu") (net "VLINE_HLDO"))
 (segment (start 24.775 18.635) (end 24.775 21.5) (width 0.25) (layer "F.Cu") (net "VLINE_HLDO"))
 (segment (start 28.125 18.635) (end 26.5 18.635) (width 0.25) (layer "F.Cu") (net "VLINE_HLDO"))
 (segment (start 37.875 21.175) (end 39 21.175) (width 0.25) (layer "F.Cu") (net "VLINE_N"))
 (via (at 39 21.175) (size 0.6) (drill 0.3) (layers "F.Cu" "B.Cu") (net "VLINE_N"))
 (segment (start 48 21.175) (end 48 17.5) (width 0.25) (layer "B.Cu") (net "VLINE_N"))
 (segment (start 39 21.175) (end 48 21.175) (width 0.25) (layer "B.Cu") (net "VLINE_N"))
 (segment (start 48 17.5) (end 53 17.5) (width 0.25) (layer "B.Cu") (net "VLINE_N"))
 (segment (start 37.875 19.905) (end 39 19.905) (width 0.25) (layer "F.Cu") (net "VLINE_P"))
 (via (at 39 19.905) (size 0.6) (drill 0.3) (layers "F.Cu" "B.Cu") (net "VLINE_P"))
 (segment (start 47 19.905) (end 47 15) (width 0.25) (layer "B.Cu") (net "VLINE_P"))
 (segment (start 47 15) (end 53 15) (width 0.25) (layer "B.Cu") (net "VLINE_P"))
 (segment (start 39 19.905) (end 47 19.905) (width 0.25) (layer "B.Cu") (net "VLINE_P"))
 (segment (start 37.875 17.365) (end 39.5 17.365) (width 0.25) (layer "F.Cu") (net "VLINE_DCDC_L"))
 (segment (start 37.875 13.555) (end 40.225 13.555) (width 0.25) (layer "F.Cu") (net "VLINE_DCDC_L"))
 (segment (start 40.225 13.555) (end 40.225 13.5) (width 0.25) (layer "F.Cu") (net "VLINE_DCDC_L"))
 (segment (start 39.5 17.365) (end 39.5 13.555) (width 0.25) (layer "F.Cu") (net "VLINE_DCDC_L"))
 (segment (start 49 27) (end 49 20) (width 0.25) (layer "F.Cu") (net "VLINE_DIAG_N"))
 (segment (start 49 20) (end 53 20) (width 0.25) (layer "F.Cu") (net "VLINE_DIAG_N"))
 (segment (start 46 16.094999) (end 46 27) (width 0.25) (layer "F.Cu") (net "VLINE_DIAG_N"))
 (segment (start 46 27) (end 44.825 27) (width 0.25) (layer "F.Cu") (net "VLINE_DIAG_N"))
 (segment (start 44.825 27) (end 49 27) (width 0.25) (layer "F.Cu") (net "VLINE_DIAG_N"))
 (segment (start 37.875 16.094999) (end 38.7 16.094999) (width 0.25) (layer "F.Cu") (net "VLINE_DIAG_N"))
 (via (at 38.7 16.094999) (size 0.6) (drill 0.3) (layers "F.Cu" "B.Cu") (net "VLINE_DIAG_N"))
 (via (at 46 16.094999) (size 0.6) (drill 0.3) (layers "F.Cu" "B.Cu") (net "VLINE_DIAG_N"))
 (segment (start 38.7 16.094999) (end 46 16.094999) (width 0.25) (layer "B.Cu") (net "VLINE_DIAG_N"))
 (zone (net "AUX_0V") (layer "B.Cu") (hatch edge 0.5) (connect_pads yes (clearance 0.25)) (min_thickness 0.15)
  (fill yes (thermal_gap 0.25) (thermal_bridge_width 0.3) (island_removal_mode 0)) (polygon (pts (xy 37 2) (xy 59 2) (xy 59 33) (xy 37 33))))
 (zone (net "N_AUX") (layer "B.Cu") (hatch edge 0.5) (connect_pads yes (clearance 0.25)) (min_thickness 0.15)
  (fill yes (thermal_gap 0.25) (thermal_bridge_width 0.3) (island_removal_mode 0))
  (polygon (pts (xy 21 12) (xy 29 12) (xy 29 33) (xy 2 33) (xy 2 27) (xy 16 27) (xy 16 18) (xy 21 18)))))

